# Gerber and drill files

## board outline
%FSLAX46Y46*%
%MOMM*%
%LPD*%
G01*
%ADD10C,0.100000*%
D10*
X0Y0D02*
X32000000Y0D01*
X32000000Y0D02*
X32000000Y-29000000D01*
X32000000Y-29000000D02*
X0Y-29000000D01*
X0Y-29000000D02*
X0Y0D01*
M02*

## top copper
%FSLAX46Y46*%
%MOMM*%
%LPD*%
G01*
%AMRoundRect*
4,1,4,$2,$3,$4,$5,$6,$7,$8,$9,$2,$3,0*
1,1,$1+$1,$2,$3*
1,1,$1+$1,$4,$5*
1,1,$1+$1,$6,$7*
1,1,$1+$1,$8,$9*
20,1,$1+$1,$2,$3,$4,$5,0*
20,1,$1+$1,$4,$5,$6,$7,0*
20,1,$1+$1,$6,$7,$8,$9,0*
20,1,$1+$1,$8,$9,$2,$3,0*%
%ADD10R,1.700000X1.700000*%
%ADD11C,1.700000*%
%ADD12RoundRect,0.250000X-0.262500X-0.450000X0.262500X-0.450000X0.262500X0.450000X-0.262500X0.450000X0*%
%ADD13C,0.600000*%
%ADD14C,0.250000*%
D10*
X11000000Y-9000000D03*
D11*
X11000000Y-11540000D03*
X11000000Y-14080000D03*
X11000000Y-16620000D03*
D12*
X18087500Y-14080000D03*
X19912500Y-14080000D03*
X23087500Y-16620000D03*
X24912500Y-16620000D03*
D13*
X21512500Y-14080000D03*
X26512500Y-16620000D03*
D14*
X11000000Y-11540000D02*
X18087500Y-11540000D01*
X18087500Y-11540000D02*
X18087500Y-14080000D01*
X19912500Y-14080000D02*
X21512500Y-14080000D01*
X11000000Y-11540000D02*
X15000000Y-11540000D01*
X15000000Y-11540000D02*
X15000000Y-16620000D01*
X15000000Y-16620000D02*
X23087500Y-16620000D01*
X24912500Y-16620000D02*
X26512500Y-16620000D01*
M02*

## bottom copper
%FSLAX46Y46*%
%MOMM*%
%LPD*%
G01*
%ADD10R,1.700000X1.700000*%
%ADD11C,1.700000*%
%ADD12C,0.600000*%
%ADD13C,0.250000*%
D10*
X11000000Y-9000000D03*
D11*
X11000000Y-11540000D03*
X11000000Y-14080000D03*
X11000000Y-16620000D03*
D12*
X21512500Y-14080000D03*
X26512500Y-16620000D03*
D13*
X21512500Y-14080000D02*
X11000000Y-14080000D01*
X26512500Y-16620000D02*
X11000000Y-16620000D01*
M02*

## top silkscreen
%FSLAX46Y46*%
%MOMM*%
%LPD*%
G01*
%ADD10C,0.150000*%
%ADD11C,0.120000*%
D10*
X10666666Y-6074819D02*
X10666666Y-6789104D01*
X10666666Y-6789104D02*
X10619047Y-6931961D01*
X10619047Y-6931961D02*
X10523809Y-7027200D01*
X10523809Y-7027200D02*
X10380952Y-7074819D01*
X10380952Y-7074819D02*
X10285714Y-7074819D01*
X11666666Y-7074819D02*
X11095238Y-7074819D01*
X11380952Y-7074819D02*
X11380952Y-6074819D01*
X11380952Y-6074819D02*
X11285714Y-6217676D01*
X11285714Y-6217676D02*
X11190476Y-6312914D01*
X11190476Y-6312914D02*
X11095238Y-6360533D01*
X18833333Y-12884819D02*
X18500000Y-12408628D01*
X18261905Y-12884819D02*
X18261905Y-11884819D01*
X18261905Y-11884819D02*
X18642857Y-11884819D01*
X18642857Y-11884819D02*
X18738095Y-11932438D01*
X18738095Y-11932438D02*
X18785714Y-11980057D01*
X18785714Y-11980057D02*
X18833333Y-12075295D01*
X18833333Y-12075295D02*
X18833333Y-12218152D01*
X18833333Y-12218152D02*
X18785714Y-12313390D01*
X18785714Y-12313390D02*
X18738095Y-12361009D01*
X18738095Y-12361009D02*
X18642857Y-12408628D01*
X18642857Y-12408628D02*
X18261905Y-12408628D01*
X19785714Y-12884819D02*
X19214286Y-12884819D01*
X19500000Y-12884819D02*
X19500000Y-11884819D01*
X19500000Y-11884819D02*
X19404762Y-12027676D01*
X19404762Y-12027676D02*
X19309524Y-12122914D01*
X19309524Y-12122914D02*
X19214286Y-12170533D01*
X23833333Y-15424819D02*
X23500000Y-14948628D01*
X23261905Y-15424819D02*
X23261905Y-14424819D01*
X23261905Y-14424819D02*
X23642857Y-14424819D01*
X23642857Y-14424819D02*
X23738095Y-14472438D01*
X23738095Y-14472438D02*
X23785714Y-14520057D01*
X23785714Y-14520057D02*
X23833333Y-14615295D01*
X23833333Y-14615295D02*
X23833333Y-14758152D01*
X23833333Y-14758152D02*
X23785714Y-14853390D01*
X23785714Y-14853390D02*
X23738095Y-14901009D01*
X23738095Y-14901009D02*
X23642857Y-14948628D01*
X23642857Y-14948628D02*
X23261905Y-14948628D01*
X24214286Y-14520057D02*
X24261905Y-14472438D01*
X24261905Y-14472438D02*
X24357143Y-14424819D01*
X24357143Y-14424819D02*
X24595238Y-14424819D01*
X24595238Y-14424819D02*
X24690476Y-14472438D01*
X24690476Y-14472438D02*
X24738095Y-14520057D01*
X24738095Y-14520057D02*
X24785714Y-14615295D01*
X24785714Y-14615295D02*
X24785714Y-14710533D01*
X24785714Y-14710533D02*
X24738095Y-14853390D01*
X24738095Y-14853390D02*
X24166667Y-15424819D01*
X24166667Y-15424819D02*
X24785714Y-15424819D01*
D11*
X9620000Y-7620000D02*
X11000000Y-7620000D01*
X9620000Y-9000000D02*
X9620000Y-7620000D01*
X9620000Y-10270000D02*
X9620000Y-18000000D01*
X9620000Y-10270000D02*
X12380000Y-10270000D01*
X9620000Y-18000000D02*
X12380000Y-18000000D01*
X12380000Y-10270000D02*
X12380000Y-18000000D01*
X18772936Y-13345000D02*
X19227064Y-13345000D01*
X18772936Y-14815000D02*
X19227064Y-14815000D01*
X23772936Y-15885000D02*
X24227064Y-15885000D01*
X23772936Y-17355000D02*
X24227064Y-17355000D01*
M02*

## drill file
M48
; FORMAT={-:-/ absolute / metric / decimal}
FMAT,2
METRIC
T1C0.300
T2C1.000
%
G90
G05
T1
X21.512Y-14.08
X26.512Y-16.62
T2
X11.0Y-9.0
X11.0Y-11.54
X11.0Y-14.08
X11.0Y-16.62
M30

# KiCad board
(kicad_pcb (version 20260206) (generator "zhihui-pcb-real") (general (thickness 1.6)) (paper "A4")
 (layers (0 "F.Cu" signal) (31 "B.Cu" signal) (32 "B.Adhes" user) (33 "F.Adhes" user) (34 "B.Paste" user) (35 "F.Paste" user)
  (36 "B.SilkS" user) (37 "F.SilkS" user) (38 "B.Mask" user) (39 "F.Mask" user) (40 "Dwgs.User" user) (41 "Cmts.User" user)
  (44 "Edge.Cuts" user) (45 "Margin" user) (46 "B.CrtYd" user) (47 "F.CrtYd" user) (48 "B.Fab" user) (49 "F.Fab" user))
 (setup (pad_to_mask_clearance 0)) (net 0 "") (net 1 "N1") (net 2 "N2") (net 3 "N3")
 (gr_line (start 0 0) (end 32 0) (stroke (width 0.1) (type default)) (layer "Edge.Cuts"))
 (gr_line (start 32 0) (end 32 29) (stroke (width 0.1) (type default)) (layer "Edge.Cuts"))
 (gr_line (start 32 29) (end 0 29) (stroke (width 0.1) (type default)) (layer "Edge.Cuts"))
 (gr_line (start 0 29) (end 0 0) (stroke (width 0.1) (type default)) (layer "Edge.Cuts"))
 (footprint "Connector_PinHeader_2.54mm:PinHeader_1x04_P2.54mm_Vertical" (layer "F.Cu")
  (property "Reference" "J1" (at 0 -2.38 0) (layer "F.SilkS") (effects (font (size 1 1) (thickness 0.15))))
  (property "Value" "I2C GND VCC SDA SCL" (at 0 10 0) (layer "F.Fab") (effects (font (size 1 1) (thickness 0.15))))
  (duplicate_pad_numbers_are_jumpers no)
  (fp_line (start -1.38 -1.38) (end 0 -1.38) (stroke (width 0.12) (type solid)) (layer "F.SilkS"))
  (fp_line (start -1.38 0) (end -1.38 -1.38) (stroke (width 0.12) (type solid)) (layer "F.SilkS"))
  (fp_line (start -1.38 1.27) (end -1.38 9) (stroke (width 0.12) (type solid)) (layer "F.SilkS"))
  (fp_line (start -1.38 1.27) (end 1.38 1.27) (stroke (width 0.12) (type solid)) (layer "F.SilkS"))
  (fp_line (start -1.38 9) (end 1.38 9) (stroke (width 0.12) (type solid)) (layer "F.SilkS"))
  (fp_line (start 1.38 1.27) (end 1.38 9) (stroke (width 0.12) (type solid)) (layer "F.SilkS"))
  (pad "1" thru_hole rect (at 0 0) (size 1.7 1.7) (drill 1) (layers "*.Cu" "*.Mask") (remove_unused_layers no))
  (pad "2" thru_hole circle (at 0 2.54) (size 1.7 1.7) (drill 1) (layers "*.Cu" "*.Mask") (remove_unused_layers no) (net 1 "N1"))
  (pad "3" thru_hole circle (at 0 5.08) (size 1.7 1.7) (drill 1) (layers "*.Cu" "*.Mask") (remove_unused_layers no) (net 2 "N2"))
  (pad "4" thru_hole circle (at 0 7.62) (size 1.7 1.7) (drill 1) (layers "*.Cu" "*.Mask") (remove_unused_layers no) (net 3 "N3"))
  (at 11 9 0))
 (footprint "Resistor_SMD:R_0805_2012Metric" (layer "F.Cu")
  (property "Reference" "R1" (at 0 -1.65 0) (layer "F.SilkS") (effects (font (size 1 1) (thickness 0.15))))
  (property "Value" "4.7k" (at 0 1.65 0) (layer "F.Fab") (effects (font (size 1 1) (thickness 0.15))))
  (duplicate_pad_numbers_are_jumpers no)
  (fp_line (start -0.227064 -0.735) (end 0.227064 -0.735) (stroke (width 0.12) (type solid)) (layer "F.SilkS"))
  (fp_line (start -0.227064 0.735) (end 0.227064 0.735) (stroke (width 0.12) (type solid)) (layer "F.SilkS"))
  (pad "1" smd roundrect (at -0.9125 0) (size 1.025 1.4) (layers "F.Cu" "F.Mask" "F.Paste") (roundrect_rratio 0.243902) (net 1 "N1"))
  (pad "2" smd roundrect (at 0.9125 0) (size 1.025 1.4) (layers "F.Cu" "F.Mask" "F.Paste") (roundrect_rratio 0.243902) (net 2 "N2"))
  (at 19 14.08 0))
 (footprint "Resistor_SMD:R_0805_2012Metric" (layer "F.Cu")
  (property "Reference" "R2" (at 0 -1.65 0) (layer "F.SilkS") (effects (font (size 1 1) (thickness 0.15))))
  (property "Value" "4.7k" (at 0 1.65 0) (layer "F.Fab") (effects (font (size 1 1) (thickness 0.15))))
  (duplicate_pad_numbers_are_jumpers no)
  (fp_line (start -0.227064 -0.735) (end 0.227064 -0.735) (stroke (width 0.12) (type solid)) (layer "F.SilkS"))
  (fp_line (start -0.227064 0.735) (end 0.227064 0.735) (stroke (width 0.12) (type solid)) (layer "F.SilkS"))
  (pad "1" smd roundrect (at -0.9125 0) (size 1.025 1.4) (layers "F.Cu" "F.Mask" "F.Paste") (roundrect_rratio 0.243902) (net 1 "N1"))
  (pad "2" smd roundrect (at 0.9125 0) (size 1.025 1.4) (layers "F.Cu" "F.Mask" "F.Paste") (roundrect_rratio 0.243902) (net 3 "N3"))
  (at 24 16.62 0))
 (segment (start 11 11.54) (end 18.0875 11.54) (width 0.25) (layer "F.Cu") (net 1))
 (segment (start 18.0875 11.54) (end 18.0875 14.08) (width 0.25) (layer "F.Cu") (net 1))
 (segment (start 19.9125 14.08) (end 21.5125 14.08) (width 0.25) (layer "F.Cu") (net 2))
 (segment (start 21.5125 14.08) (end 11 14.08) (width 0.25) (layer "B.Cu") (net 2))
 (segment (start 11 11.54) (end 15 11.54) (width 0.25) (layer "F.Cu") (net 1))
 (segment (start 15 11.54) (end 15 16.62) (width 0.25) (layer "F.Cu") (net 1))
 (segment (start 15 16.62) (end 23.0875 16.62) (width 0.25) (layer "F.Cu") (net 1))
 (segment (start 24.9125 16.62) (end 26.5125 16.62) (width 0.25) (layer "F.Cu") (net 3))
 (segment (start 26.5125 16.62) (end 11 16.62) (width 0.25) (layer "B.Cu") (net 3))
 (via (at 21.5125 14.08) (size 0.6) (drill 0.3) (layers "F.Cu" "B.Cu") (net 2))
 (via (at 26.5125 16.62) (size 0.6) (drill 0.3) (layers "F.Cu" "B.Cu") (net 3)))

